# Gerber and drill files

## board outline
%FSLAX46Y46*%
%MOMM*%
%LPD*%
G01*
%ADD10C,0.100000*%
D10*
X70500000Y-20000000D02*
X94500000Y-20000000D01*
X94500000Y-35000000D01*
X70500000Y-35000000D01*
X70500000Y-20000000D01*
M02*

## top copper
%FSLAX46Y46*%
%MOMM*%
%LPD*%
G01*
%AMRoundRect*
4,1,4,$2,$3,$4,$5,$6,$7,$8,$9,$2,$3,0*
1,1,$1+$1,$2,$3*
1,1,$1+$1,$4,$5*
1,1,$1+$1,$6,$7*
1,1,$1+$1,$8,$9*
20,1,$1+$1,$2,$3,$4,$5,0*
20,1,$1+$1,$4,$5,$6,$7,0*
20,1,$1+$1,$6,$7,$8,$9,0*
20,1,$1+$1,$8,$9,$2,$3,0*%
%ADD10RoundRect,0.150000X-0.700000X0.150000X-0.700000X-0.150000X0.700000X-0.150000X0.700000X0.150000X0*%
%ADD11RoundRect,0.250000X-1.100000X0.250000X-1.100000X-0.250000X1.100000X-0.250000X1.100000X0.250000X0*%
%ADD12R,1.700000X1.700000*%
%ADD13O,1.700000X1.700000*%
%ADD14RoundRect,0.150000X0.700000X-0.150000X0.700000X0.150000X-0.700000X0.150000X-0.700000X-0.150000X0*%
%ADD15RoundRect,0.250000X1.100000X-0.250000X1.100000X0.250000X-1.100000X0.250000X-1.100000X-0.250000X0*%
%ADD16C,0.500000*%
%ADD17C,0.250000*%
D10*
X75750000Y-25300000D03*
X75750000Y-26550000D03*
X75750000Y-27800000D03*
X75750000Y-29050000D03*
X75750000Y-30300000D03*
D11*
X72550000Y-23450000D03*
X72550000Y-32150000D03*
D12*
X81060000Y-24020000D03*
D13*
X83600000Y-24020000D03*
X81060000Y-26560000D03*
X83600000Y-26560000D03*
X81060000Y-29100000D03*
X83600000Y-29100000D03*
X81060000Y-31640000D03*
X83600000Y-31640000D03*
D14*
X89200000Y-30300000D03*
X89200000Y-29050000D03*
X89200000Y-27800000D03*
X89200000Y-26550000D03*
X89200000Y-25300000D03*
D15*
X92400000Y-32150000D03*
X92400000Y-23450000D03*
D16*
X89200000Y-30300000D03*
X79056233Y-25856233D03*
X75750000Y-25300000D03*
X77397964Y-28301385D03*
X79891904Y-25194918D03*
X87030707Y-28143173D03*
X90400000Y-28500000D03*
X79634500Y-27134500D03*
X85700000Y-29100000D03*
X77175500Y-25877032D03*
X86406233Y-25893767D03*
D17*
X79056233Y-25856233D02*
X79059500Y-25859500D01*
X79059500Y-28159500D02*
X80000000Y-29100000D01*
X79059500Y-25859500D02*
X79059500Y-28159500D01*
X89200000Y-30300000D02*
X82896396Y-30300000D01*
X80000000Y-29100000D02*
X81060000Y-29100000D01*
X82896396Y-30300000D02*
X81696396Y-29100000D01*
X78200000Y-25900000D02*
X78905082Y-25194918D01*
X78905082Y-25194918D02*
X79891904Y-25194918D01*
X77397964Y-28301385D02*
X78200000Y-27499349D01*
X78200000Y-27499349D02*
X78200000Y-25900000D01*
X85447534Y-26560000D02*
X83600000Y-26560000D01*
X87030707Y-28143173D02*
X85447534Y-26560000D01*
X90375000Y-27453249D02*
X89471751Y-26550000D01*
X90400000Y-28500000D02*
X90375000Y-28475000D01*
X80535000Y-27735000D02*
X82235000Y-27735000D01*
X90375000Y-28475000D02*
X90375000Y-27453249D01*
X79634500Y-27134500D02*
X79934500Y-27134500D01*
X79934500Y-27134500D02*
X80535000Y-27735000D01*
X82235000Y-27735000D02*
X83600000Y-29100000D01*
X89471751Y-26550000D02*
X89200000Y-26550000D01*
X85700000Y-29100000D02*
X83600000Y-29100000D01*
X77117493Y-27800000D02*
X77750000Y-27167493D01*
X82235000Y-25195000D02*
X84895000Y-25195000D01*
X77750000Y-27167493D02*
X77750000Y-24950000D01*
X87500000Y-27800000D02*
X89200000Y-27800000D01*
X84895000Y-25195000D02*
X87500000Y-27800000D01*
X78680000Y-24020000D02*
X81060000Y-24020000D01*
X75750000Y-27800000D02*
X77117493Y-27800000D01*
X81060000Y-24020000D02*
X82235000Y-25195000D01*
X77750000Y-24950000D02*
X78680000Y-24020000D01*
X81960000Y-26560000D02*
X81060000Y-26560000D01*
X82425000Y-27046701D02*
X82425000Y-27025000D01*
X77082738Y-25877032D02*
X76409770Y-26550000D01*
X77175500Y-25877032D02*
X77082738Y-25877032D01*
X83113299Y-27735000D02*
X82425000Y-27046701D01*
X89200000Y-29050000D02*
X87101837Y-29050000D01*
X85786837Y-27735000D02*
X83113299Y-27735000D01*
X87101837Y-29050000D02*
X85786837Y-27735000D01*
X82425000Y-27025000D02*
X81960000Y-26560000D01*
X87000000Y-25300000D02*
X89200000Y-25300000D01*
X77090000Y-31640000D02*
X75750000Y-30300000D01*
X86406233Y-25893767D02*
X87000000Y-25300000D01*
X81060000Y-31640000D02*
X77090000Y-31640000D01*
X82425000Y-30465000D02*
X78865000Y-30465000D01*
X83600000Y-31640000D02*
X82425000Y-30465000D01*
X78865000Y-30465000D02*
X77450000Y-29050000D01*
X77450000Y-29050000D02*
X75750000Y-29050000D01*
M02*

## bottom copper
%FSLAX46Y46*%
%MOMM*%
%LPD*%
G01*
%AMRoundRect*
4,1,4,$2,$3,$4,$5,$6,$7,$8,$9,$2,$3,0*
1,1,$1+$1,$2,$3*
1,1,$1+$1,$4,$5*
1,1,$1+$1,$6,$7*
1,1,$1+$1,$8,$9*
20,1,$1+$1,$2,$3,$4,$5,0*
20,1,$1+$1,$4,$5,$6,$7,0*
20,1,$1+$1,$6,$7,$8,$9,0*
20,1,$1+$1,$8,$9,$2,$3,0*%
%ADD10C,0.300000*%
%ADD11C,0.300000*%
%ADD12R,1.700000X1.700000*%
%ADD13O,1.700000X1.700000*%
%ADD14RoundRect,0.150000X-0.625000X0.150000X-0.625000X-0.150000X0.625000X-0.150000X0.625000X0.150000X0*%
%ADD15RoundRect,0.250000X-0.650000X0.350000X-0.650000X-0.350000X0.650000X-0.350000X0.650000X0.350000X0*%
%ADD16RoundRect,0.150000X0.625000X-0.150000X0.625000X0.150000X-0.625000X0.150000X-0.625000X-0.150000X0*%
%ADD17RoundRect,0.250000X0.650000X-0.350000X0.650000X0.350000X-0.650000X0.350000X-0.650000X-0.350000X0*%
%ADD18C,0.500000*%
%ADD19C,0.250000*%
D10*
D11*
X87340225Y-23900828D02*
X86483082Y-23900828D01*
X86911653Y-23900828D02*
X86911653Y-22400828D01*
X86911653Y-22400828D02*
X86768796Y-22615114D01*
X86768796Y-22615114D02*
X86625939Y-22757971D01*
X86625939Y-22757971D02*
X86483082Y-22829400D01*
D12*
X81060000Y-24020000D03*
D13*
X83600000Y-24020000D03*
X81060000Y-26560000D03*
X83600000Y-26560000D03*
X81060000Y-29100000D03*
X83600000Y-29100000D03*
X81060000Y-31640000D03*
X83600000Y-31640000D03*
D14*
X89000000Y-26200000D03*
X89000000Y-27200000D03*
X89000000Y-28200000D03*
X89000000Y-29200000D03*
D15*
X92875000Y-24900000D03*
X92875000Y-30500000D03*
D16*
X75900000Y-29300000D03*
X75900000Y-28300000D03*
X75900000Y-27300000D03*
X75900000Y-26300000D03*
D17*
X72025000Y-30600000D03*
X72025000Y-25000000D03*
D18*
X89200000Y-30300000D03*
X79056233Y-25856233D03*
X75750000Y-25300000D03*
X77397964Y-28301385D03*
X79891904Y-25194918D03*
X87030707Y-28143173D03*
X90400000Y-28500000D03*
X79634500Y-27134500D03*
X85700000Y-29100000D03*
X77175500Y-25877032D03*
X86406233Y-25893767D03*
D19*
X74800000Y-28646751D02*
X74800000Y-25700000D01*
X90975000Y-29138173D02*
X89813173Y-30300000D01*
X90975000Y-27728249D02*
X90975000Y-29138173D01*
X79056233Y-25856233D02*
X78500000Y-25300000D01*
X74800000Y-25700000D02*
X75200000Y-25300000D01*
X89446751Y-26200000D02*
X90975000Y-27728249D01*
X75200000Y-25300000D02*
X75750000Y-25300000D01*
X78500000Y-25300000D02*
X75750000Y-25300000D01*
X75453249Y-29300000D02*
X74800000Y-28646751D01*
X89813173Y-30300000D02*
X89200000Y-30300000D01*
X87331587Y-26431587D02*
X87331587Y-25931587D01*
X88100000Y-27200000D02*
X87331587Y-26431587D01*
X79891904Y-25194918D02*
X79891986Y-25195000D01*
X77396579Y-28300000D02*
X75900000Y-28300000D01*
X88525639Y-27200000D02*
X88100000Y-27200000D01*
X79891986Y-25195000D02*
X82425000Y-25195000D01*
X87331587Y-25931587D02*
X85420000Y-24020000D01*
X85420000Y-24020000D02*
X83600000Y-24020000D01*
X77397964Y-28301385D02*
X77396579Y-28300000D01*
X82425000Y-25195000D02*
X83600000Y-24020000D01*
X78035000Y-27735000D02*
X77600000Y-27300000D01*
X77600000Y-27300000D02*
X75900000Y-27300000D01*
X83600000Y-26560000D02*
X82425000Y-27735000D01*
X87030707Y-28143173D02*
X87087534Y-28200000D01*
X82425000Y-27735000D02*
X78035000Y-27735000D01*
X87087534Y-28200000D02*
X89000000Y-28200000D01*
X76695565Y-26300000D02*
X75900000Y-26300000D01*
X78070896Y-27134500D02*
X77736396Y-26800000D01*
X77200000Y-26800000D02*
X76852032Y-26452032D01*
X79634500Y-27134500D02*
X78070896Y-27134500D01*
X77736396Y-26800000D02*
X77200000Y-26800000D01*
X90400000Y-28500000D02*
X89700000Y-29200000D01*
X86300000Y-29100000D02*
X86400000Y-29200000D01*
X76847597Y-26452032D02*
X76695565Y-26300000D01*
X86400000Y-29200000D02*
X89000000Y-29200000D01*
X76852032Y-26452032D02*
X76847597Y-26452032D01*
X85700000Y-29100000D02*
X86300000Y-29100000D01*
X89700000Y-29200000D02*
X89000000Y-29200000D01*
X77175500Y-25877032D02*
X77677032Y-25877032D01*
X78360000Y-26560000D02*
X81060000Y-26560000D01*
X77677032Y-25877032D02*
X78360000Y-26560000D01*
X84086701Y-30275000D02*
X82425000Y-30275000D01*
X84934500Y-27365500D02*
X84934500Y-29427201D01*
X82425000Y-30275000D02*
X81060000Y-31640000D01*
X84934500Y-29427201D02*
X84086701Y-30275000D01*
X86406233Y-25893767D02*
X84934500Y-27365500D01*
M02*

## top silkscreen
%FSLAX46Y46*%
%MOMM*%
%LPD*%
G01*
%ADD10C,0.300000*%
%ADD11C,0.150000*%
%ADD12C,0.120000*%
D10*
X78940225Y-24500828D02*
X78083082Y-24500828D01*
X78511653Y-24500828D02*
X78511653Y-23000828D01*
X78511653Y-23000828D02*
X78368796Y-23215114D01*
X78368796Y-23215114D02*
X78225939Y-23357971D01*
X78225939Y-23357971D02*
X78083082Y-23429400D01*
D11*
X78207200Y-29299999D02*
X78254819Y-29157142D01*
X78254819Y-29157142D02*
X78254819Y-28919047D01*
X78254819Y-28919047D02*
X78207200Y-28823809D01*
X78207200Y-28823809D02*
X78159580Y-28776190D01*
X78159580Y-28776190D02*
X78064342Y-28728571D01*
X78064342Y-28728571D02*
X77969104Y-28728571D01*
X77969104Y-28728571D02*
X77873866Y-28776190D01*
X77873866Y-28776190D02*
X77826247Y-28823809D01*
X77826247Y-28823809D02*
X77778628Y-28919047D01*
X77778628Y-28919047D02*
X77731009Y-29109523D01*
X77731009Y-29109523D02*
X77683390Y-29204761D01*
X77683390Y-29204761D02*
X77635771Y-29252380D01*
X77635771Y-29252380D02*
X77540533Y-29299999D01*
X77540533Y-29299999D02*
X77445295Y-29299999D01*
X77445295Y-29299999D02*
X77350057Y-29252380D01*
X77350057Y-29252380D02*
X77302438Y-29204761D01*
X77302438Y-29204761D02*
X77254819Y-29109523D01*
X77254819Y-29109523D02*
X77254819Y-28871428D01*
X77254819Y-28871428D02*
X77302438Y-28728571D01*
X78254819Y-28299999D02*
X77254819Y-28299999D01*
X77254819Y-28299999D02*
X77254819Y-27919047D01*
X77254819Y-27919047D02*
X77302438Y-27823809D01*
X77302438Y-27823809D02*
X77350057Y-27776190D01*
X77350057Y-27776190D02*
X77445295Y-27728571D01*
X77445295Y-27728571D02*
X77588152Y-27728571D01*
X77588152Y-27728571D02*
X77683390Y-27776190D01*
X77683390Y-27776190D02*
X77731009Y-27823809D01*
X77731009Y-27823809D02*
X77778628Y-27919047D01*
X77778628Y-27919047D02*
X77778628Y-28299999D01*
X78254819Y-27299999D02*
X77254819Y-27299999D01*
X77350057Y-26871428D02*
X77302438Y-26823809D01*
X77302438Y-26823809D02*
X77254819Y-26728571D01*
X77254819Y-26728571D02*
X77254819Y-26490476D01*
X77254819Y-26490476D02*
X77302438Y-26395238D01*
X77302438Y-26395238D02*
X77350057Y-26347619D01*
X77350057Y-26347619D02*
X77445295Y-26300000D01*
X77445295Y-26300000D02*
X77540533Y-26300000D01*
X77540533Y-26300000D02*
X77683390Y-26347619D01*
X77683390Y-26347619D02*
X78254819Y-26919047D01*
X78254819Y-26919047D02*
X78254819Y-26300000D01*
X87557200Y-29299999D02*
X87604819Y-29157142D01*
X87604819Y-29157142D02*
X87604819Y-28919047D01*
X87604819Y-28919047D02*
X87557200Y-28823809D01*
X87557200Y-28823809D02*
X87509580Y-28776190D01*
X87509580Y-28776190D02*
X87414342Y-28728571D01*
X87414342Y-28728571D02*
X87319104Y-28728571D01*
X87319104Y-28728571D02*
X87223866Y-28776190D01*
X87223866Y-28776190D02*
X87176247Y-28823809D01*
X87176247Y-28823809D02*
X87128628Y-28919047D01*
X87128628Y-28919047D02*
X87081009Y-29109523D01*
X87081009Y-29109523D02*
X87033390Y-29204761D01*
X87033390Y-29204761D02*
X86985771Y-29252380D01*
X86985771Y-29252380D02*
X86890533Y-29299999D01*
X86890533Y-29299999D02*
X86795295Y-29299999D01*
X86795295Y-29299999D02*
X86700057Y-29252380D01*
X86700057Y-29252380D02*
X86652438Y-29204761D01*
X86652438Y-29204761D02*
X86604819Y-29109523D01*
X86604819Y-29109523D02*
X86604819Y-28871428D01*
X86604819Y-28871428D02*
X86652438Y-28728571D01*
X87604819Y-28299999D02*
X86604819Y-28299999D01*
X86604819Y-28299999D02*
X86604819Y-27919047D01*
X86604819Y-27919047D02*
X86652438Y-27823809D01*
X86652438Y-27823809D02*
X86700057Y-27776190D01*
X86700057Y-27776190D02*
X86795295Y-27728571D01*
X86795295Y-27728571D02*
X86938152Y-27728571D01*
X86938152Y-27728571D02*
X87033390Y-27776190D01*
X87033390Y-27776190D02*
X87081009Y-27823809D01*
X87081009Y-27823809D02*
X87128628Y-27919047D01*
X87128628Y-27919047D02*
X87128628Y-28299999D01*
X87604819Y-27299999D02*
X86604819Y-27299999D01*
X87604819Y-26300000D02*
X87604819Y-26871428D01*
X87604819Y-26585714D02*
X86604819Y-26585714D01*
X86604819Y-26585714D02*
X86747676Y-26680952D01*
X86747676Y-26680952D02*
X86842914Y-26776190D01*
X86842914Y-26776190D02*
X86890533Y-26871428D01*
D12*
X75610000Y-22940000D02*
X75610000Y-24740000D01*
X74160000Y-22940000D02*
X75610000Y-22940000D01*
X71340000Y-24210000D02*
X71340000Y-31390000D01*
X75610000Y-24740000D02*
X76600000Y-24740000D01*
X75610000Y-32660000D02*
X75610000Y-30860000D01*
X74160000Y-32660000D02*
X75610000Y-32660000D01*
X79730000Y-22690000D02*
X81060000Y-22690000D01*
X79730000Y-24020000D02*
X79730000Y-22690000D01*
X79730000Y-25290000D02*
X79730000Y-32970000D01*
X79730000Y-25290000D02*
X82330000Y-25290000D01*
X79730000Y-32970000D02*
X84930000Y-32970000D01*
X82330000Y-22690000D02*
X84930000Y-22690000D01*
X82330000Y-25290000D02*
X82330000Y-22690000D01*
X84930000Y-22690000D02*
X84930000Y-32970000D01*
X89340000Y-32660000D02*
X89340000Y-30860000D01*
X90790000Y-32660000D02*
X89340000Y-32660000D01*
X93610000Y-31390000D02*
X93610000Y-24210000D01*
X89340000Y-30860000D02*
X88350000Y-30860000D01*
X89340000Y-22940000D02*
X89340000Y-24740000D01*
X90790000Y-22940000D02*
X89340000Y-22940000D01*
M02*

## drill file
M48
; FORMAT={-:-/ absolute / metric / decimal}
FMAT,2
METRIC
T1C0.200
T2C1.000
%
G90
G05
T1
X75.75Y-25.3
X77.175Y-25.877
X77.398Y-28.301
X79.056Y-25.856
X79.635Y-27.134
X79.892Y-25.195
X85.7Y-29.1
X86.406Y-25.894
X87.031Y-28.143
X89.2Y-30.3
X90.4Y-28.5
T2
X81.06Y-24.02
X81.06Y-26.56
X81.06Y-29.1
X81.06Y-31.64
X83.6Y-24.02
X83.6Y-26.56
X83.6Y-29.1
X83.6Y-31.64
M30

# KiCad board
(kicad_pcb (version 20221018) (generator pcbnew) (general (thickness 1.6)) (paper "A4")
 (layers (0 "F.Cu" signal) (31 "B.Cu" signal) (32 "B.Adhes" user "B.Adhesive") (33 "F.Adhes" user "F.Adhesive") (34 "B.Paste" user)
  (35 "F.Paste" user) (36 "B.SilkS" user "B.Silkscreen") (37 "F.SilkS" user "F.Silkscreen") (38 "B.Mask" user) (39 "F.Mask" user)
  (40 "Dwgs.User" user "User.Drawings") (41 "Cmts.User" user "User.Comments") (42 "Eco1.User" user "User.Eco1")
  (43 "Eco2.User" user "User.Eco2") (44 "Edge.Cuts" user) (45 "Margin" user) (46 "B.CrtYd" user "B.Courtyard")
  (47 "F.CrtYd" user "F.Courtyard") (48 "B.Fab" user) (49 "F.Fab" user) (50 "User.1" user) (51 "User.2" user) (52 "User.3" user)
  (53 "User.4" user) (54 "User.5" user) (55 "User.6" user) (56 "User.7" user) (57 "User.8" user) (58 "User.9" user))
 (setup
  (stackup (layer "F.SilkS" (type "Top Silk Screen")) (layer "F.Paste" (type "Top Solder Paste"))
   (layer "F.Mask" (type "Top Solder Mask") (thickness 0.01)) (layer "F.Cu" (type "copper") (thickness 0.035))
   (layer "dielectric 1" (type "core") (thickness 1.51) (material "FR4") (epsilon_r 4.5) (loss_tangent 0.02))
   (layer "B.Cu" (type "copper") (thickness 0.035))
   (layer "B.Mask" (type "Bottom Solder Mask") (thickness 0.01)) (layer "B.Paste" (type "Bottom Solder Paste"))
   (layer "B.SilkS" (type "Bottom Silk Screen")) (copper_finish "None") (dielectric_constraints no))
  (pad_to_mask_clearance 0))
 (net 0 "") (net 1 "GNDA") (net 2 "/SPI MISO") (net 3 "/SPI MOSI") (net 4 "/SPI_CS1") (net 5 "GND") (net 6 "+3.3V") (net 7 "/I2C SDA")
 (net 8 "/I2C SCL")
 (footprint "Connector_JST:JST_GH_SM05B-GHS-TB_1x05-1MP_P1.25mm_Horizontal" (layer "F.Cu") (at 73.9 27.8 -90)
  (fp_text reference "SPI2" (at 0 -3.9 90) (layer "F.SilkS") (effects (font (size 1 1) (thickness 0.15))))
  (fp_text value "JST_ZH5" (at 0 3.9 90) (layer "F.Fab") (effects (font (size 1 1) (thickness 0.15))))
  (fp_line (start -4.86 -1.71) (end -3.06 -1.71) (stroke (width 0.12) (type solid)) (layer "F.SilkS"))
  (fp_line (start -4.86 -0.26) (end -4.86 -1.71) (stroke (width 0.12) (type solid)) (layer "F.SilkS"))
  (fp_line (start -3.59 2.56) (end 3.59 2.56) (stroke (width 0.12) (type solid)) (layer "F.SilkS"))
  (fp_line (start -3.06 -1.71) (end -3.06 -2.7) (stroke (width 0.12) (type solid)) (layer "F.SilkS"))
  (fp_line (start 4.86 -1.71) (end 3.06 -1.71) (stroke (width 0.12) (type solid)) (layer "F.SilkS"))
  (fp_line (start 4.86 -0.26) (end 4.86 -1.71) (stroke (width 0.12) (type solid)) (layer "F.SilkS"))
  (pad "1" smd roundrect (at -2.5 -1.85 270) (size 0.6 1.7) (layers "F.Cu" "F.Paste" "F.Mask") (roundrect_rratio 0.25) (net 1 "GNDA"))
  (pad "2" smd roundrect (at -1.25 -1.85 270) (size 0.6 1.7) (layers "F.Cu" "F.Paste" "F.Mask") (roundrect_rratio 0.25) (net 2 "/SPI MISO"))
  (pad "3" smd roundrect (at 0 -1.85 270) (size 0.6 1.7) (layers "F.Cu" "F.Paste" "F.Mask") (roundrect_rratio 0.25) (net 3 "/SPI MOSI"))
  (pad "4" smd roundrect (at 1.25 -1.85 270) (size 0.6 1.7) (layers "F.Cu" "F.Paste" "F.Mask") (roundrect_rratio 0.25) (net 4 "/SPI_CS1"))
  (pad "5" smd roundrect (at 2.5 -1.85 270) (size 0.6 1.7) (layers "F.Cu" "F.Paste" "F.Mask") (roundrect_rratio 0.25) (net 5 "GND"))
  (pad "MP" smd roundrect (at -4.35 1.35 270) (size 1 2.7) (layers "F.Cu" "F.Paste" "F.Mask") (roundrect_rratio 0.25))
  (pad "MP" smd roundrect (at 4.35 1.35 270) (size 1 2.7) (layers "F.Cu" "F.Paste" "F.Mask") (roundrect_rratio 0.25)))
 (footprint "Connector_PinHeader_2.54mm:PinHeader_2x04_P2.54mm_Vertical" (layer "F.Cu") (at 81.06 24.02)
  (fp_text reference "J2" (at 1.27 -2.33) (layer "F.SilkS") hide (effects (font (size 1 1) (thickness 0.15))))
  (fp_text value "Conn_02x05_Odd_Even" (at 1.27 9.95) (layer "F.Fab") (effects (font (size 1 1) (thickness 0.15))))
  (fp_line (start -1.33 -1.33) (end 0 -1.33) (stroke (width 0.12) (type solid)) (layer "F.SilkS"))
  (fp_line (start -1.33 0) (end -1.33 -1.33) (stroke (width 0.12) (type solid)) (layer "F.SilkS"))
  (fp_line (start -1.33 1.27) (end -1.33 8.95) (stroke (width 0.12) (type solid)) (layer "F.SilkS"))
  (fp_line (start -1.33 1.27) (end 1.27 1.27) (stroke (width 0.12) (type solid)) (layer "F.SilkS"))
  (fp_line (start -1.33 8.95) (end 3.87 8.95) (stroke (width 0.12) (type solid)) (layer "F.SilkS"))
  (fp_line (start 1.27 -1.33) (end 3.87 -1.33) (stroke (width 0.12) (type solid)) (layer "F.SilkS"))
  (fp_line (start 1.27 1.27) (end 1.27 -1.33) (stroke (width 0.12) (type solid)) (layer "F.SilkS"))
  (fp_line (start 3.87 -1.33) (end 3.87 8.95) (stroke (width 0.12) (type solid)) (layer "F.SilkS"))
  (pad "1" thru_hole rect (at 0 0) (size 1.7 1.7) (drill 1) (layers "*.Cu" "*.Mask") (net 3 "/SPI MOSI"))
  (pad "2" thru_hole oval (at 2.54 0) (size 1.7 1.7) (drill 1) (layers "*.Cu" "*.Mask") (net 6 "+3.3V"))
  (pad "3" thru_hole oval (at 0 2.54) (size 1.7 1.7) (drill 1) (layers "*.Cu" "*.Mask") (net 2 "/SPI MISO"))
  (pad "4" thru_hole oval (at 2.54 2.54) (size 1.7 1.7) (drill 1) (layers "*.Cu" "*.Mask") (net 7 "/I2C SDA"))
  (pad "5" thru_hole oval (at 0 5.08) (size 1.7 1.7) (drill 1) (layers "*.Cu" "*.Mask") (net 1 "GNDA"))
  (pad "6" thru_hole oval (at 2.54 5.08) (size 1.7 1.7) (drill 1) (layers "*.Cu" "*.Mask") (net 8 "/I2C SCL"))
  (pad "7" thru_hole oval (at 0 7.62) (size 1.7 1.7) (drill 1) (layers "*.Cu" "*.Mask") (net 5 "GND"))
  (pad "8" thru_hole oval (at 2.54 7.62) (size 1.7 1.7) (drill 1) (layers "*.Cu" "*.Mask") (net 4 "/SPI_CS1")))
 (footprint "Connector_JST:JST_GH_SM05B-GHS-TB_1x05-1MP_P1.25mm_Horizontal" (layer "F.Cu") (at 91.05 27.8 90)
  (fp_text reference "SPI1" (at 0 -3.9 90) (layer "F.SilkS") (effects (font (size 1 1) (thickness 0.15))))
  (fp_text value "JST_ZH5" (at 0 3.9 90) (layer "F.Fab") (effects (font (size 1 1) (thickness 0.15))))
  (fp_line (start -4.86 -1.71) (end -3.06 -1.71) (stroke (width 0.12) (type solid)) (layer "F.SilkS"))
  (fp_line (start -4.86 -0.26) (end -4.86 -1.71) (stroke (width 0.12) (type solid)) (layer "F.SilkS"))
  (fp_line (start -3.59 2.56) (end 3.59 2.56) (stroke (width 0.12) (type solid)) (layer "F.SilkS"))
  (fp_line (start -3.06 -1.71) (end -3.06 -2.7) (stroke (width 0.12) (type solid)) (layer "F.SilkS"))
  (fp_line (start 4.86 -1.71) (end 3.06 -1.71) (stroke (width 0.12) (type solid)) (layer "F.SilkS"))
  (fp_line (start 4.86 -0.26) (end 4.86 -1.71) (stroke (width 0.12) (type solid)) (layer "F.SilkS"))
  (pad "1" smd roundrect (at -2.5 -1.85 90) (size 0.6 1.7) (layers "F.Cu" "F.Paste" "F.Mask") (roundrect_rratio 0.25) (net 1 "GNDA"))
  (pad "2" smd roundrect (at -1.25 -1.85 90) (size 0.6 1.7) (layers "F.Cu" "F.Paste" "F.Mask") (roundrect_rratio 0.25) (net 2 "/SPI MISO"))
  (pad "3" smd roundrect (at 0 -1.85 90) (size 0.6 1.7) (layers "F.Cu" "F.Paste" "F.Mask") (roundrect_rratio 0.25) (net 3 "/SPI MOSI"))
  (pad "4" smd roundrect (at 1.25 -1.85 90) (size 0.6 1.7) (layers "F.Cu" "F.Paste" "F.Mask") (roundrect_rratio 0.25) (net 8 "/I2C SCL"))
  (pad "5" smd roundrect (at 2.5 -1.85 90) (size 0.6 1.7) (layers "F.Cu" "F.Paste" "F.Mask") (roundrect_rratio 0.25) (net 5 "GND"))
  (pad "MP" smd roundrect (at -4.35 1.35 90) (size 1 2.7) (layers "F.Cu" "F.Paste" "F.Mask") (roundrect_rratio 0.25))
  (pad "MP" smd roundrect (at 4.35 1.35 90) (size 1 2.7) (layers "F.Cu" "F.Paste" "F.Mask") (roundrect_rratio 0.25)))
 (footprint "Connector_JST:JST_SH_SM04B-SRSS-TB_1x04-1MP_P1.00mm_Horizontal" (layer "B.Cu") (at 91 27.7 -90)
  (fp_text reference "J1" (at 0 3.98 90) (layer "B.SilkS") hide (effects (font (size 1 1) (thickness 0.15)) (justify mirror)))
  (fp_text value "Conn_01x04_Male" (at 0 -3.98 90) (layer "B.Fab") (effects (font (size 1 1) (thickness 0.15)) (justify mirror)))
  (pad "1" smd roundrect (at -1.5 2 270) (size 0.6 1.55) (layers "B.Cu" "B.Paste" "B.Mask") (roundrect_rratio 0.25) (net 1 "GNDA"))
  (pad "2" smd roundrect (at -0.5 2 270) (size 0.6 1.55) (layers "B.Cu" "B.Paste" "B.Mask") (roundrect_rratio 0.25) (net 6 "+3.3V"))
  (pad "3" smd roundrect (at 0.5 2 270) (size 0.6 1.55) (layers "B.Cu" "B.Paste" "B.Mask") (roundrect_rratio 0.25) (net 7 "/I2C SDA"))
  (pad "4" smd roundrect (at 1.5 2 270) (size 0.6 1.55) (layers "B.Cu" "B.Paste" "B.Mask") (roundrect_rratio 0.25) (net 8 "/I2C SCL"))
  (pad "MP" smd roundrect (at -2.8 -1.875 270) (size 1.2 1.8) (layers "B.Cu" "B.Paste" "B.Mask") (roundrect_rratio 0.208333))
  (pad "MP" smd roundrect (at 2.8 -1.875 270) (size 1.2 1.8) (layers "B.Cu" "B.Paste" "B.Mask") (roundrect_rratio 0.208333)))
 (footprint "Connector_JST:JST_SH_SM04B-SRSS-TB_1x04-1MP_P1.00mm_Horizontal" (layer "B.Cu") (at 73.9 27.8 90)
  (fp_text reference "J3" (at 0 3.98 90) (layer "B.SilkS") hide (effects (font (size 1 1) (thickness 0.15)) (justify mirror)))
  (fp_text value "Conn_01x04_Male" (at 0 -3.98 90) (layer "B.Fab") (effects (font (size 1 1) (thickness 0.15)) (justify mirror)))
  (pad "1" smd roundrect (at -1.5 2 90) (size 0.6 1.55) (layers "B.Cu" "B.Paste" "B.Mask") (roundrect_rratio 0.25) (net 1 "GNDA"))
  (pad "2" smd roundrect (at -0.5 2 90) (size 0.6 1.55) (layers "B.Cu" "B.Paste" "B.Mask") (roundrect_rratio 0.25) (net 6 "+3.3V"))
  (pad "3" smd roundrect (at 0.5 2 90) (size 0.6 1.55) (layers "B.Cu" "B.Paste" "B.Mask") (roundrect_rratio 0.25) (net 7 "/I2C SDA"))
  (pad "4" smd roundrect (at 1.5 2 90) (size 0.6 1.55) (layers "B.Cu" "B.Paste" "B.Mask") (roundrect_rratio 0.25) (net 8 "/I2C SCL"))
  (pad "MP" smd roundrect (at -2.8 -1.875 90) (size 1.2 1.8) (layers "B.Cu" "B.Paste" "B.Mask") (roundrect_rratio 0.208333))
  (pad "MP" smd roundrect (at 2.8 -1.875 90) (size 1.2 1.8) (layers "B.Cu" "B.Paste" "B.Mask") (roundrect_rratio 0.208333)))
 (gr_rect (start 70.5 20) (end 94.5 35) (stroke (width 0.1) (type default)) (fill none) (layer "Edge.Cuts"))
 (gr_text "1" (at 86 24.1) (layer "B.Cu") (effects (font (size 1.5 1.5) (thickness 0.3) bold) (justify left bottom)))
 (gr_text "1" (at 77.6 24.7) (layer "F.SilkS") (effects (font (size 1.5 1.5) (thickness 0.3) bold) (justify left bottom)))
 (segment (start 79.056233 25.856233) (end 79.0595 25.8595) (width 0.25) (layer "F.Cu") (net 1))
 (segment (start 79.0595 28.1595) (end 80 29.1) (width 0.25) (layer "F.Cu") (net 1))
 (segment (start 79.0595 25.8595) (end 79.0595 28.1595) (width 0.25) (layer "F.Cu") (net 1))
 (segment (start 89.2 30.3) (end 82.896396 30.3) (width 0.25) (layer "F.Cu") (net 1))
 (segment (start 80 29.1) (end 81.06 29.1) (width 0.25) (layer "F.Cu") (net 1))
 (segment (start 82.896396 30.3) (end 81.696396 29.1) (width 0.25) (layer "F.Cu") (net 1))
 (via (at 89.2 30.3) (size 0.5) (drill 0.2) (layers "F.Cu" "B.Cu") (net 1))
 (via (at 79.056233 25.856233) (size 0.5) (drill 0.2) (layers "F.Cu" "B.Cu") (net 1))
 (via (at 75.75 25.3) (size 0.5) (drill 0.2) (layers "F.Cu" "B.Cu") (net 1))
 (segment (start 74.8 28.646751) (end 74.8 25.7) (width 0.25) (layer "B.Cu") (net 1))
 (segment (start 90.975 29.138173) (end 89.813173 30.3) (width 0.25) (layer "B.Cu") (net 1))
 (segment (start 90.975 27.728249) (end 90.975 29.138173) (width 0.25) (layer "B.Cu") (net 1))
 (segment (start 79.056233 25.856233) (end 78.5 25.3) (width 0.25) (layer "B.Cu") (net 1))
 (segment (start 74.8 25.7) (end 75.2 25.3) (width 0.25) (layer "B.Cu") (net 1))
 (segment (start 89.446751 26.2) (end 90.975 27.728249) (width 0.25) (layer "B.Cu") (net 1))
 (segment (start 75.2 25.3) (end 75.75 25.3) (width 0.25) (layer "B.Cu") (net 1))
 (segment (start 78.5 25.3) (end 75.75 25.3) (width 0.25) (layer "B.Cu") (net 1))
 (segment (start 75.453249 29.3) (end 74.8 28.646751) (width 0.25) (layer "B.Cu") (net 1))
 (segment (start 89.813173 30.3) (end 89.2 30.3) (width 0.25) (layer "B.Cu") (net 1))
 (segment (start 78.2 25.9) (end 78.905082 25.194918) (width 0.25) (layer "F.Cu") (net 6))
 (segment (start 78.905082 25.194918) (end 79.891904 25.194918) (width 0.25) (layer "F.Cu") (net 6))
 (segment (start 77.397964 28.301385) (end 78.2 27.499349) (width 0.25) (layer "F.Cu") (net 6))
 (segment (start 78.2 27.499349) (end 78.2 25.9) (width 0.25) (layer "F.Cu") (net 6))
 (via (at 77.397964 28.301385) (size 0.5) (drill 0.2) (layers "F.Cu" "B.Cu") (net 6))
 (via (at 79.891904 25.194918) (size 0.5) (drill 0.2) (layers "F.Cu" "B.Cu") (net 6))
 (segment (start 87.331587 26.431587) (end 87.331587 25.931587) (width 0.25) (layer "B.Cu") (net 6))
 (segment (start 88.1 27.2) (end 87.331587 26.431587) (width 0.25) (layer "B.Cu") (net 6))
 (segment (start 79.891904 25.194918) (end 79.891986 25.195) (width 0.25) (layer "B.Cu") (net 6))
 (segment (start 77.396579 28.3) (end 75.9 28.3) (width 0.25) (layer "B.Cu") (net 6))
 (segment (start 88.525639 27.2) (end 88.1 27.2) (width 0.25) (layer "B.Cu") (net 6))
 (segment (start 79.891986 25.195) (end 82.425 25.195) (width 0.25) (layer "B.Cu") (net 6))
 (segment (start 87.331587 25.931587) (end 85.42 24.02) (width 0.25) (layer "B.Cu") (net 6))
 (segment (start 85.42 24.02) (end 83.6 24.02) (width 0.25) (layer "B.Cu") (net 6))
 (segment (start 77.397964 28.301385) (end 77.396579 28.3) (width 0.25) (layer "B.Cu") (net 6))
 (segment (start 82.425 25.195) (end 83.6 24.02) (width 0.25) (layer "B.Cu") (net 6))
 (segment (start 85.447534 26.56) (end 83.6 26.56) (width 0.25) (layer "F.Cu") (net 7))
 (segment (start 87.030707 28.143173) (end 85.447534 26.56) (width 0.25) (layer "F.Cu") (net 7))
 (via (at 87.030707 28.143173) (size 0.5) (drill 0.2) (layers "F.Cu" "B.Cu") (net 7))
 (segment (start 78.035 27.735) (end 77.6 27.3) (width 0.25) (layer "B.Cu") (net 7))
 (segment (start 77.6 27.3) (end 75.9 27.3) (width 0.25) (layer "B.Cu") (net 7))
 (segment (start 83.6 26.56) (end 82.425 27.735) (width 0.25) (layer "B.Cu") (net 7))
 (segment (start 87.030707 28.143173) (end 87.087534 28.2) (width 0.25) (layer "B.Cu") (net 7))
 (segment (start 82.425 27.735) (end 78.035 27.735) (width 0.25) (layer "B.Cu") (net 7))
 (segment (start 87.087534 28.2) (end 89 28.2) (width 0.25) (layer "B.Cu") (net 7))
 (segment (start 90.375 27.453249) (end 89.471751 26.55) (width 0.25) (layer "F.Cu") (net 8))
 (segment (start 90.4 28.5) (end 90.375 28.475) (width 0.25) (layer "F.Cu") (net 8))
 (segment (start 80.535 27.735) (end 82.235 27.735) (width 0.25) (layer "F.Cu") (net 8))
 (segment (start 90.375 28.475) (end 90.375 27.453249) (width 0.25) (layer "F.Cu") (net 8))
 (segment (start 79.6345 27.1345) (end 79.9345 27.1345) (width 0.25) (layer "F.Cu") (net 8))
 (segment (start 79.9345 27.1345) (end 80.535 27.735) (width 0.25) (layer "F.Cu") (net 8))
 (segment (start 82.235 27.735) (end 83.6 29.1) (width 0.25) (layer "F.Cu") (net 8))
 (segment (start 89.471751 26.55) (end 89.2 26.55) (width 0.25) (layer "F.Cu") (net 8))
 (segment (start 85.7 29.1) (end 83.6 29.1) (width 0.25) (layer "F.Cu") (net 8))
 (via (at 90.4 28.5) (size 0.5) (drill 0.2) (layers "F.Cu" "B.Cu") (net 8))
 (via (at 79.6345 27.1345) (size 0.5) (drill 0.2) (layers "F.Cu" "B.Cu") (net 8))
 (via (at 85.7 29.1) (size 0.5) (drill 0.2) (layers "F.Cu" "B.Cu") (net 8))
 (segment (start 76.695565 26.3) (end 75.9 26.3) (width 0.25) (layer "B.Cu") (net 8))
 (segment (start 78.070896 27.1345) (end 77.736396 26.8) (width 0.25) (layer "B.Cu") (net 8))
 (segment (start 77.2 26.8) (end 76.852032 26.452032) (width 0.25) (layer "B.Cu") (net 8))
 (segment (start 79.6345 27.1345) (end 78.070896 27.1345) (width 0.25) (layer "B.Cu") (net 8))
 (segment (start 77.736396 26.8) (end 77.2 26.8) (width 0.25) (layer "B.Cu") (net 8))
 (segment (start 90.4 28.5) (end 89.7 29.2) (width 0.25) (layer "B.Cu") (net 8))
 (segment (start 86.3 29.1) (end 86.4 29.2) (width 0.25) (layer "B.Cu") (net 8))
 (segment (start 76.847597 26.452032) (end 76.695565 26.3) (width 0.25) (layer "B.Cu") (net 8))
 (segment (start 86.4 29.2) (end 89 29.2) (width 0.25) (layer "B.Cu") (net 8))
 (segment (start 76.852032 26.452032) (end 76.847597 26.452032) (width 0.25) (layer "B.Cu") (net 8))
 (segment (start 85.7 29.1) (end 86.3 29.1) (width 0.25) (layer "B.Cu") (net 8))
 (segment (start 89.7 29.2) (end 89 29.2) (width 0.25) (layer "B.Cu") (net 8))
 (segment (start 77.117493 27.8) (end 77.75 27.167493) (width 0.25) (layer "F.Cu") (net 3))
 (segment (start 82.235 25.195) (end 84.895 25.195) (width 0.25) (layer "F.Cu") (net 3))
 (segment (start 77.75 27.167493) (end 77.75 24.95) (width 0.25) (layer "F.Cu") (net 3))
 (segment (start 87.5 27.8) (end 89.2 27.8) (width 0.25) (layer "F.Cu") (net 3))
 (segment (start 84.895 25.195) (end 87.5 27.8) (width 0.25) (layer "F.Cu") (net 3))
 (segment (start 78.68 24.02) (end 81.06 24.02) (width 0.25) (layer "F.Cu") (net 3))
 (segment (start 75.75 27.8) (end 77.117493 27.8) (width 0.25) (layer "F.Cu") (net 3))
 (segment (start 81.06 24.02) (end 82.235 25.195) (width 0.25) (layer "F.Cu") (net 3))
 (segment (start 77.75 24.95) (end 78.68 24.02) (width 0.25) (layer "F.Cu") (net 3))
 (segment (start 81.96 26.56) (end 81.06 26.56) (width 0.25) (layer "F.Cu") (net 2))
 (segment (start 82.425 27.046701) (end 82.425 27.025) (width 0.25) (layer "F.Cu") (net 2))
 (segment (start 77.082738 25.877032) (end 76.40977 26.55) (width 0.25) (layer "F.Cu") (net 2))
 (segment (start 77.1755 25.877032) (end 77.082738 25.877032) (width 0.25) (layer "F.Cu") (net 2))
 (segment (start 83.113299 27.735) (end 82.425 27.046701) (width 0.25) (layer "F.Cu") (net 2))
 (segment (start 89.2 29.05) (end 87.101837 29.05) (width 0.25) (layer "F.Cu") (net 2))
 (segment (start 85.786837 27.735) (end 83.113299 27.735) (width 0.25) (layer "F.Cu") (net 2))
 (segment (start 87.101837 29.05) (end 85.786837 27.735) (width 0.25) (layer "F.Cu") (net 2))
 (segment (start 82.425 27.025) (end 81.96 26.56) (width 0.25) (layer "F.Cu") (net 2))
 (via (at 77.1755 25.877032) (size 0.5) (drill 0.2) (layers "F.Cu" "B.Cu") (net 2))
 (segment (start 77.1755 25.877032) (end 77.677032 25.877032) (width 0.25) (layer "B.Cu") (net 2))
 (segment (start 78.36 26.56) (end 81.06 26.56) (width 0.25) (layer "B.Cu") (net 2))
 (segment (start 77.677032 25.877032) (end 78.36 26.56) (width 0.25) (layer "B.Cu") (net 2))
 (segment (start 87 25.3) (end 89.2 25.3) (width 0.25) (layer "F.Cu") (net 5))
 (segment (start 77.09 31.64) (end 75.75 30.3) (width 0.25) (layer "F.Cu") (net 5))
 (segment (start 86.406233 25.893767) (end 87 25.3) (width 0.25) (layer "F.Cu") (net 5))
 (segment (start 81.06 31.64) (end 77.09 31.64) (width 0.25) (layer "F.Cu") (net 5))
 (via (at 86.406233 25.893767) (size 0.5) (drill 0.2) (layers "F.Cu" "B.Cu") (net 5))
 (segment (start 84.086701 30.275) (end 82.425 30.275) (width 0.25) (layer "B.Cu") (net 5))
 (segment (start 84.9345 27.3655) (end 84.9345 29.427201) (width 0.25) (layer "B.Cu") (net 5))
 (segment (start 82.425 30.275) (end 81.06 31.64) (width 0.25) (layer "B.Cu") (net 5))
 (segment (start 84.9345 29.427201) (end 84.086701 30.275) (width 0.25) (layer "B.Cu") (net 5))
 (segment (start 86.406233 25.893767) (end 84.9345 27.3655) (width 0.25) (layer "B.Cu") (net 5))
 (segment (start 82.425 30.465) (end 78.865 30.465) (width 0.25) (layer "F.Cu") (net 4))
 (segment (start 83.6 31.64) (end 82.425 30.465) (width 0.25) (layer "F.Cu") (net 4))
 (segment (start 78.865 30.465) (end 77.45 29.05) (width 0.25) (layer "F.Cu") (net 4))
 (segment (start 77.45 29.05) (end 75.75 29.05) (width 0.25) (layer "F.Cu") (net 4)))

